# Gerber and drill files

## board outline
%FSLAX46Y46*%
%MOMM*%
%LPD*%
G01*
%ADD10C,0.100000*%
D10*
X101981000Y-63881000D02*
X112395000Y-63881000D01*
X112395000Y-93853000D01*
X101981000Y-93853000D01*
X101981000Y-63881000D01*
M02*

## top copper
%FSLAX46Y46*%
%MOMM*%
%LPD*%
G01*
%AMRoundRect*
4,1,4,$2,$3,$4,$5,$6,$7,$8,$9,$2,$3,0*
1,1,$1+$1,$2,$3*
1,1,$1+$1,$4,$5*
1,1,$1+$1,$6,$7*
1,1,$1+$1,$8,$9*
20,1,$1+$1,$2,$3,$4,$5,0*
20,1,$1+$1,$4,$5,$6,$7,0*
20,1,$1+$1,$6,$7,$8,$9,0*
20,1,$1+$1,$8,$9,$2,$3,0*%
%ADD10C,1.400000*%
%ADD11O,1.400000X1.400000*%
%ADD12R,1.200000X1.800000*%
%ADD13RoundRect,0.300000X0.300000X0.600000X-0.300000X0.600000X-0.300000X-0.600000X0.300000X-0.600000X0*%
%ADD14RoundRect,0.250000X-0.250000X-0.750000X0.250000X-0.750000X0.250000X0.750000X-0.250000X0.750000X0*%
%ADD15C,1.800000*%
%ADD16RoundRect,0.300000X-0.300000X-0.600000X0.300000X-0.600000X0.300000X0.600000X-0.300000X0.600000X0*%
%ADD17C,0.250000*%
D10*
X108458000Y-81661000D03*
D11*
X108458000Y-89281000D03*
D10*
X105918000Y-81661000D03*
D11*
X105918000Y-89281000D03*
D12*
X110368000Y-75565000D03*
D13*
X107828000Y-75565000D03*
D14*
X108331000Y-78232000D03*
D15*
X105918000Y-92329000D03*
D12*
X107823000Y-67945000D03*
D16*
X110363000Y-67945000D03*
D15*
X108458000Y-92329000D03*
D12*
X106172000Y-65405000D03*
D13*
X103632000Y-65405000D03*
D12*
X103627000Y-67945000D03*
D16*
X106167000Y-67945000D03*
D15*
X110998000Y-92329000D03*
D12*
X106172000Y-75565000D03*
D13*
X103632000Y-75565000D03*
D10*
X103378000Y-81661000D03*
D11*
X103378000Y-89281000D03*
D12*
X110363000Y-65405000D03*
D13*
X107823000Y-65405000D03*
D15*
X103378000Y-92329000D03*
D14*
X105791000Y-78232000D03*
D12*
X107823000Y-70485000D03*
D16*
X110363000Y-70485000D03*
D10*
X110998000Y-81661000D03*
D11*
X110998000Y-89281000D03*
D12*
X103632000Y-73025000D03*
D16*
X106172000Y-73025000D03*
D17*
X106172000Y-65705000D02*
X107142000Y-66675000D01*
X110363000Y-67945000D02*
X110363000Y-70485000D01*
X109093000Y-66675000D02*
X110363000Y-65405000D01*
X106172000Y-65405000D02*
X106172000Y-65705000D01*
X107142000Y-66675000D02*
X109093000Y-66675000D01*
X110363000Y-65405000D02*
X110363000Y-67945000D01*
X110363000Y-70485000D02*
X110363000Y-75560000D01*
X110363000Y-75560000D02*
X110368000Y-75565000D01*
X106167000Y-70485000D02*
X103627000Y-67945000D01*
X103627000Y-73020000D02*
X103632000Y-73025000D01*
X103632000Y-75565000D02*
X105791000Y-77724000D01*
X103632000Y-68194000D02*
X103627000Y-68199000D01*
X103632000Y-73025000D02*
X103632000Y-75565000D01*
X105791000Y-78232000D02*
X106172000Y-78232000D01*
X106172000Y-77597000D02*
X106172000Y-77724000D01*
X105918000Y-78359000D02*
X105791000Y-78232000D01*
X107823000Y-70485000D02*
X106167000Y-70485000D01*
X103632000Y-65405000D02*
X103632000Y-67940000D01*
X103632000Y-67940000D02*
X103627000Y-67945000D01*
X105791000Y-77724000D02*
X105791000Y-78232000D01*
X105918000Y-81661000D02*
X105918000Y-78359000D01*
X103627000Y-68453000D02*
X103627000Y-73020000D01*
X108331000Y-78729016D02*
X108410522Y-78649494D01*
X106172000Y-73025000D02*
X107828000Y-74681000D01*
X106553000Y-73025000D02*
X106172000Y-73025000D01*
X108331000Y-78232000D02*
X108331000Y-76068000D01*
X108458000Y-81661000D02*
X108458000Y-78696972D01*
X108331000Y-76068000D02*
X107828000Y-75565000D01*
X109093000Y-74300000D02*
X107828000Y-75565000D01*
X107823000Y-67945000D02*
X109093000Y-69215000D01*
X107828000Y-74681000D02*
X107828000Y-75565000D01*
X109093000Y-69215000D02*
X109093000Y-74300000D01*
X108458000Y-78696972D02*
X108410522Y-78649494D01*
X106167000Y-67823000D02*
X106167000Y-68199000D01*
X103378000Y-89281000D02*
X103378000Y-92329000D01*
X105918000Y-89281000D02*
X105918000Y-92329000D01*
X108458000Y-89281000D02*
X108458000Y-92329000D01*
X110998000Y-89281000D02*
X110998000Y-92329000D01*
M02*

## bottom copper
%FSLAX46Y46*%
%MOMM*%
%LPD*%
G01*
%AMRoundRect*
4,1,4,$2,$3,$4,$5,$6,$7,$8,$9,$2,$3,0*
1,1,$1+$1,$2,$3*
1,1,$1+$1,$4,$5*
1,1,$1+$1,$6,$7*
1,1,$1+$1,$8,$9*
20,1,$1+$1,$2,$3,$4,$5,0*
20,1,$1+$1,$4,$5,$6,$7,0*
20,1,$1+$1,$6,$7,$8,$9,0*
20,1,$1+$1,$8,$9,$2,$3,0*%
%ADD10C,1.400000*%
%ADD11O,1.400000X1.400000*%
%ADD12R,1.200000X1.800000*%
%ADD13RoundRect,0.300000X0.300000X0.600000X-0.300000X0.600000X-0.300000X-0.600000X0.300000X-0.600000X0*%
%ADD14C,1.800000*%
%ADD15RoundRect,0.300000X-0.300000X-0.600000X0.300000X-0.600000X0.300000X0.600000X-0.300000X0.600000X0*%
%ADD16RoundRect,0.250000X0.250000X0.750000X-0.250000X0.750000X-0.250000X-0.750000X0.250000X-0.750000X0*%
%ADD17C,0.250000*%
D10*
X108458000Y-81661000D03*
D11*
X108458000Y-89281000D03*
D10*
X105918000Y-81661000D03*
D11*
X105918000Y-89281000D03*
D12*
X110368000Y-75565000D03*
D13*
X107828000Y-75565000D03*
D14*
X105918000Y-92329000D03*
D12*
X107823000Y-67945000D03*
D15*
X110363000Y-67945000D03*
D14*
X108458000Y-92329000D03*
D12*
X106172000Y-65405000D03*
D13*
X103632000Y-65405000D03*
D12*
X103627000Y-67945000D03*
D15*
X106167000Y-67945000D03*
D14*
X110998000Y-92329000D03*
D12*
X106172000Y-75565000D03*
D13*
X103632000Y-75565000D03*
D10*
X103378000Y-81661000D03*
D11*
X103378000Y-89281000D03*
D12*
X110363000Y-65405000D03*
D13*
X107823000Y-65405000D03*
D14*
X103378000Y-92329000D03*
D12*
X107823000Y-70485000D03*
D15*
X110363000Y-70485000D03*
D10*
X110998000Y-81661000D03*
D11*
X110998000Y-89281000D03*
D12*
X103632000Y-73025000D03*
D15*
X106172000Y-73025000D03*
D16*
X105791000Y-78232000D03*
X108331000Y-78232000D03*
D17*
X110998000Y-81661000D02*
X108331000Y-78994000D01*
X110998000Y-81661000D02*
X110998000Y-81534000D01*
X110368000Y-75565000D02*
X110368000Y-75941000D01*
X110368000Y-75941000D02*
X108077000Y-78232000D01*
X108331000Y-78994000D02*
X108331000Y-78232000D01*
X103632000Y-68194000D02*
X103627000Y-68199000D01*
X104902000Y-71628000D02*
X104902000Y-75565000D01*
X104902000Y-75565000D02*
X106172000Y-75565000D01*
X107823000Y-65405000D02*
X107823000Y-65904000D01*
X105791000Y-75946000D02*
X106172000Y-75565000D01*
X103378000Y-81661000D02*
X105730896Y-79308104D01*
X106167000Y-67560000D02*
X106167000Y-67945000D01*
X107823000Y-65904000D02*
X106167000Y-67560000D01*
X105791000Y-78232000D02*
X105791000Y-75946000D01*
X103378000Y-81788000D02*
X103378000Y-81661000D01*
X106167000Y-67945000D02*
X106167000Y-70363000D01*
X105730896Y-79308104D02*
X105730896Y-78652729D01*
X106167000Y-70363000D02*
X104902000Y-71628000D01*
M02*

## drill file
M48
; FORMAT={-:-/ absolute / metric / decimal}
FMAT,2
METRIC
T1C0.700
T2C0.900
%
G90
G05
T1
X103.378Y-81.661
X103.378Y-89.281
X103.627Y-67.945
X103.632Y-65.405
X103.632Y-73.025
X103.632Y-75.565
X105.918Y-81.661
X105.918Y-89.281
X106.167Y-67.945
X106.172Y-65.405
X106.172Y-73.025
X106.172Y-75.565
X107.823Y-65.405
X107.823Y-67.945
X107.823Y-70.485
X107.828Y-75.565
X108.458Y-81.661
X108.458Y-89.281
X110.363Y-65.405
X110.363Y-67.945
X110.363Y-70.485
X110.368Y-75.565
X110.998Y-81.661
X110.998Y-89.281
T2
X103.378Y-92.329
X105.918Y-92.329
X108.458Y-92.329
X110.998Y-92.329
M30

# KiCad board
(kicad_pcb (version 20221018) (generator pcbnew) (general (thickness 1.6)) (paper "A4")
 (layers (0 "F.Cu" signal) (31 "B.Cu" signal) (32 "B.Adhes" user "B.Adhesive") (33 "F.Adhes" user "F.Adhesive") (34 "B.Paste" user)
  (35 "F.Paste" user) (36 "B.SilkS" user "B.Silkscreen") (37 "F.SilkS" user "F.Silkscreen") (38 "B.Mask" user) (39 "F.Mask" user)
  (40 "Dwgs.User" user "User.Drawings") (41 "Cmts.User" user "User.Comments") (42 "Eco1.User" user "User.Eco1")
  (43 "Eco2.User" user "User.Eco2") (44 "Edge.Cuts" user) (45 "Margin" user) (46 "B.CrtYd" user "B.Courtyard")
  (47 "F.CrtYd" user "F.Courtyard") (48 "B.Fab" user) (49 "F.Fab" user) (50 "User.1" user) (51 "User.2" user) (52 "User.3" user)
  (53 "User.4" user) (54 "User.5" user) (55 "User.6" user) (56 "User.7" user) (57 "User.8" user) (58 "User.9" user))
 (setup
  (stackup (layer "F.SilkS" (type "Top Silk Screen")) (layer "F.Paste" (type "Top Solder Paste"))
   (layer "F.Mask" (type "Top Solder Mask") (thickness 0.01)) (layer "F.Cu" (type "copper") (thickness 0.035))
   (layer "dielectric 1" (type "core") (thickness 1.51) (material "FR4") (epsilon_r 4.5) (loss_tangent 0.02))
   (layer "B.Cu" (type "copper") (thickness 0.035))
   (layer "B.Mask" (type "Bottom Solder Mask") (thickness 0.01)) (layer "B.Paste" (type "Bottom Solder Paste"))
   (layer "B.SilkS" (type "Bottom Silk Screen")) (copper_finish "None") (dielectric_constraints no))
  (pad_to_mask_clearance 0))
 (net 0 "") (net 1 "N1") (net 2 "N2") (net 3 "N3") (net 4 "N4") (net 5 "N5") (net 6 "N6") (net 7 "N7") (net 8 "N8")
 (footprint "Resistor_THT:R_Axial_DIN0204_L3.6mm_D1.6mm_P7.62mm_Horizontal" (layer "F.Cu") (at 108.458 81.661 -90)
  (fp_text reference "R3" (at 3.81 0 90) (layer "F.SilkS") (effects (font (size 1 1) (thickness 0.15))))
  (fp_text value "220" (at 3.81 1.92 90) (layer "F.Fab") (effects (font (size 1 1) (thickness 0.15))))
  (pad "1" thru_hole circle (at 0 0 270) (size 1.4 1.4) (drill 0.7) (layers "*.Cu" "*.Mask") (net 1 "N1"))
  (pad "2" thru_hole oval (at 7.62 0 270) (size 1.4 1.4) (drill 0.7) (layers "*.Cu" "*.Mask") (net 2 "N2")))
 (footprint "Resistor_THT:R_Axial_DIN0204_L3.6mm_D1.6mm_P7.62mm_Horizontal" (layer "F.Cu") (at 105.918 81.661 -90)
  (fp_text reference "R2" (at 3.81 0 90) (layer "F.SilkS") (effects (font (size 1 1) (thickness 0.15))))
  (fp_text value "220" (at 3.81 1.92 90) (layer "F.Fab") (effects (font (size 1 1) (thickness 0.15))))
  (pad "1" thru_hole circle (at 0 0 270) (size 1.4 1.4) (drill 0.7) (layers "*.Cu" "*.Mask") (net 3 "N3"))
  (pad "2" thru_hole oval (at 7.62 0 270) (size 1.4 1.4) (drill 0.7) (layers "*.Cu" "*.Mask") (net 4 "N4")))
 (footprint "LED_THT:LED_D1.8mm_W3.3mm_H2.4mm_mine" (layer "F.Cu") (at 110.368 75.565 180)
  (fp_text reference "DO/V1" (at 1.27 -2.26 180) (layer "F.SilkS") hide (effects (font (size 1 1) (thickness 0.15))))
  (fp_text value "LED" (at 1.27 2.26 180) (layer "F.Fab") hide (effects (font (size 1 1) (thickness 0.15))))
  (pad "1" thru_hole rect (at 0 0 180) (size 1.2 1.8) (drill 0.7) (layers "*.Cu" "*.Mask") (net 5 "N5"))
  (pad "2" thru_hole roundrect (at 2.54 0 180) (size 1.2 1.8) (drill 0.7) (layers "*.Cu" "*.Mask") (roundrect_rratio 0.25) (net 1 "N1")))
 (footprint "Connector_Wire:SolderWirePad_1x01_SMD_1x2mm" (layer "F.Cu") (at 108.331 78.232)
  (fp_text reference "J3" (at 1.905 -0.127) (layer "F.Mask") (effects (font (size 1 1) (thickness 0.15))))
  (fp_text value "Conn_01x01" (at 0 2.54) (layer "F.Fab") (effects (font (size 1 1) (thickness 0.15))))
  (pad "1" smd roundrect (at 0 0) (size 1 2) (layers "F.Cu" "F.Paste" "F.Mask") (roundrect_rratio 0.25) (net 1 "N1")))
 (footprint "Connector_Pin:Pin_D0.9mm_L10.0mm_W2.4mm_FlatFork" (layer "F.Cu") (at 105.918 92.329)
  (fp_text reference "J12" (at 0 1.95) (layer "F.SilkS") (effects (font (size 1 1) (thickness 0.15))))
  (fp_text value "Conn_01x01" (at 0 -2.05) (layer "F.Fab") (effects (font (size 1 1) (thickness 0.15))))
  (pad "1" thru_hole circle (at 0 0) (size 1.8 1.8) (drill 0.9) (layers "*.Cu" "*.Mask") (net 4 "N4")))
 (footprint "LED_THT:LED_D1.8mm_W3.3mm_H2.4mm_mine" (layer "F.Cu") (at 107.823 67.945)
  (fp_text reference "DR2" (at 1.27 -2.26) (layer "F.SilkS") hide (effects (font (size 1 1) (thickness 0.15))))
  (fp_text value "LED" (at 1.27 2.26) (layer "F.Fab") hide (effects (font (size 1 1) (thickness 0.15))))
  (pad "1" thru_hole rect (at 0 0) (size 1.2 1.8) (drill 0.7) (layers "*.Cu" "*.Mask") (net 1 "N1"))
  (pad "2" thru_hole roundrect (at 2.54 0) (size 1.2 1.8) (drill 0.7) (layers "*.Cu" "*.Mask") (roundrect_rratio 0.25) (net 5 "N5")))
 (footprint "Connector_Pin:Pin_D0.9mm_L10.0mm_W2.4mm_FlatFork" (layer "F.Cu") (at 108.458 92.329)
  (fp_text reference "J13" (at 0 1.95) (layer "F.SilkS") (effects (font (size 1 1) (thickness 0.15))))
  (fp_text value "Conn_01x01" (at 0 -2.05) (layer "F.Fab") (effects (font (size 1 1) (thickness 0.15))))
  (pad "1" thru_hole circle (at 0 0) (size 1.8 1.8) (drill 0.9) (layers "*.Cu" "*.Mask") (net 2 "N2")))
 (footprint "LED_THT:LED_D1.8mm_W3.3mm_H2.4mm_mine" (layer "F.Cu") (at 106.172 65.405 180)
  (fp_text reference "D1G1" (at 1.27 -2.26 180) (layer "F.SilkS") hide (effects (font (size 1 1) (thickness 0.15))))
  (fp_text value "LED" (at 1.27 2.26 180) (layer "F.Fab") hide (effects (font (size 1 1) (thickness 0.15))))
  (pad "1" thru_hole rect (at 0 0 180) (size 1.2 1.8) (drill 0.7) (layers "*.Cu" "*.Mask") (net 5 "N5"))
  (pad "2" thru_hole roundrect (at 2.54 0 180) (size 1.2 1.8) (drill 0.7) (layers "*.Cu" "*.Mask") (roundrect_rratio 0.25) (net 3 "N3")))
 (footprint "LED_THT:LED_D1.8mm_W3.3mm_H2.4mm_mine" (layer "F.Cu") (at 103.627 67.945)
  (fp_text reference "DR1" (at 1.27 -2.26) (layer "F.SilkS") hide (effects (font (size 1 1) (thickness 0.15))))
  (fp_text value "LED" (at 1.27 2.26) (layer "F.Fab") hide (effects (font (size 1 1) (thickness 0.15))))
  (pad "1" thru_hole rect (at 0 0) (size 1.2 1.8) (drill 0.7) (layers "*.Cu" "*.Mask") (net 3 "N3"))
  (pad "2" thru_hole roundrect (at 2.54 0) (size 1.2 1.8) (drill 0.7) (layers "*.Cu" "*.Mask") (roundrect_rratio 0.25) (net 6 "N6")))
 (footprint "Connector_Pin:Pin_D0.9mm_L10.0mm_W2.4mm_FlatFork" (layer "F.Cu") (at 110.998 92.329)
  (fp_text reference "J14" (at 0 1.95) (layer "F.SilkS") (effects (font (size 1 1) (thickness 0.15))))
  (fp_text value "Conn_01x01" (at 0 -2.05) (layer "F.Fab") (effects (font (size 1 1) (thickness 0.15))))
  (pad "1" thru_hole circle (at 0 0) (size 1.8 1.8) (drill 0.9) (layers "*.Cu" "*.Mask") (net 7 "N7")))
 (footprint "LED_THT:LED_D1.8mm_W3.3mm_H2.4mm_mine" (layer "F.Cu") (at 106.172 75.565 180)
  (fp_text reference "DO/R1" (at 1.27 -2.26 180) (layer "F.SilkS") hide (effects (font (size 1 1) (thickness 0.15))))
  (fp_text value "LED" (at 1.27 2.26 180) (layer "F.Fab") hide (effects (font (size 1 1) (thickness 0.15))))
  (pad "1" thru_hole rect (at 0 0 180) (size 1.2 1.8) (drill 0.7) (layers "*.Cu" "*.Mask") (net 6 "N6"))
  (pad "2" thru_hole roundrect (at 2.54 0 180) (size 1.2 1.8) (drill 0.7) (layers "*.Cu" "*.Mask") (roundrect_rratio 0.25) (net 3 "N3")))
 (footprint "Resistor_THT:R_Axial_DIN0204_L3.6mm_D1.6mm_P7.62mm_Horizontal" (layer "F.Cu") (at 103.378 81.661 -90)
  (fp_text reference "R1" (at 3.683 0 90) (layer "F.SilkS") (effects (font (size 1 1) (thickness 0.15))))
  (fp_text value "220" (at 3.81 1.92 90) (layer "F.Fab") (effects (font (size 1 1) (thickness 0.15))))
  (pad "1" thru_hole circle (at 0 0 270) (size 1.4 1.4) (drill 0.7) (layers "*.Cu" "*.Mask") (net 6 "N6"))
  (pad "2" thru_hole oval (at 7.62 0 270) (size 1.4 1.4) (drill 0.7) (layers "*.Cu" "*.Mask") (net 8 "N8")))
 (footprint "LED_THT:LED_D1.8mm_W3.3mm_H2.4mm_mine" (layer "F.Cu") (at 110.363 65.405 180)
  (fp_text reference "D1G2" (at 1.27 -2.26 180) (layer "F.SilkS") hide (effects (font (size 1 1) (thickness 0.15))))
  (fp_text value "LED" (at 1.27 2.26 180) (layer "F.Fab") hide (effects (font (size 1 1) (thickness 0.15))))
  (pad "1" thru_hole rect (at 0 0 180) (size 1.2 1.8) (drill 0.7) (layers "*.Cu" "*.Mask") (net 5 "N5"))
  (pad "2" thru_hole roundrect (at 2.54 0 180) (size 1.2 1.8) (drill 0.7) (layers "*.Cu" "*.Mask") (roundrect_rratio 0.25) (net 6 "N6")))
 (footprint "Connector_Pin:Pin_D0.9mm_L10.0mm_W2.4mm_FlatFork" (layer "F.Cu") (at 103.378 92.329)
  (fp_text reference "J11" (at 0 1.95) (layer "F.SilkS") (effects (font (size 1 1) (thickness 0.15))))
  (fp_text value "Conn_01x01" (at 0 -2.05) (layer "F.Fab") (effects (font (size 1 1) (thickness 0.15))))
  (pad "1" thru_hole circle (at 0 0) (size 1.8 1.8) (drill 0.9) (layers "*.Cu" "*.Mask") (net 8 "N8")))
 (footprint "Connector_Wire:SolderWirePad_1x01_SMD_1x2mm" (layer "F.Cu") (at 105.791 78.232)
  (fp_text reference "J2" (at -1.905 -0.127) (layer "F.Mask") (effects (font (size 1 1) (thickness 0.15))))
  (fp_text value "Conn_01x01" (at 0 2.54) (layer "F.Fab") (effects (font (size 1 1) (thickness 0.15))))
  (pad "1" smd roundrect (at 0 0) (size 1 2) (layers "F.Cu" "F.Paste" "F.Mask") (roundrect_rratio 0.25) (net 3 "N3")))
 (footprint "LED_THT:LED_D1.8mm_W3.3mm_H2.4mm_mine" (layer "F.Cu") (at 107.823 70.485)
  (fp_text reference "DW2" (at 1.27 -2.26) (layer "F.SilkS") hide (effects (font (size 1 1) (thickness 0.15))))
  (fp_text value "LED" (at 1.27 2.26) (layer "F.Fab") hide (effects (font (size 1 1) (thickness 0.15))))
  (pad "1" thru_hole rect (at 0 0) (size 1.2 1.8) (drill 0.7) (layers "*.Cu" "*.Mask") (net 3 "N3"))
  (pad "2" thru_hole roundrect (at 2.54 0) (size 1.2 1.8) (drill 0.7) (layers "*.Cu" "*.Mask") (roundrect_rratio 0.25) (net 5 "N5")))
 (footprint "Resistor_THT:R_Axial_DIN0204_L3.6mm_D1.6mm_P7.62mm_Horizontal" (layer "F.Cu") (at 110.998 81.661 -90)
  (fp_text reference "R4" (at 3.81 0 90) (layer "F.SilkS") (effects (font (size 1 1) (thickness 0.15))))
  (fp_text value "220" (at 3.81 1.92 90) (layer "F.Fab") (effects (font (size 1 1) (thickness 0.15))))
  (pad "1" thru_hole circle (at 0 0 270) (size 1.4 1.4) (drill 0.7) (layers "*.Cu" "*.Mask") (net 5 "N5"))
  (pad "2" thru_hole oval (at 7.62 0 270) (size 1.4 1.4) (drill 0.7) (layers "*.Cu" "*.Mask") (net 7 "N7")))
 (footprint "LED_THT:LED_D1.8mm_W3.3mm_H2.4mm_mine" (layer "F.Cu") (at 103.632 73.025)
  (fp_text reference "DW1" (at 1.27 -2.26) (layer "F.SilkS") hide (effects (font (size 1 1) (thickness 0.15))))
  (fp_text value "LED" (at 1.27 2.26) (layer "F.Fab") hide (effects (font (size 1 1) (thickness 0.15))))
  (pad "1" thru_hole rect (at 0 0) (size 1.2 1.8) (drill 0.7) (layers "*.Cu" "*.Mask") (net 3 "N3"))
  (pad "2" thru_hole roundrect (at 2.54 0) (size 1.2 1.8) (drill 0.7) (layers "*.Cu" "*.Mask") (roundrect_rratio 0.25) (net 1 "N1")))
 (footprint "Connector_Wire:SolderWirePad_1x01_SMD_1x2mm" (layer "B.Cu") (at 105.791 78.232 180)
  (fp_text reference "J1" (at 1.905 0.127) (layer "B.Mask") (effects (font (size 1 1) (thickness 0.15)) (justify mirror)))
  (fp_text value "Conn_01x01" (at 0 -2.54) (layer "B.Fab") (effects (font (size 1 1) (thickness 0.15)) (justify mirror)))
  (pad "1" smd roundrect (at 0 0 180) (size 1 2) (layers "B.Cu" "B.Paste" "B.Mask") (roundrect_rratio 0.25) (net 6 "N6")))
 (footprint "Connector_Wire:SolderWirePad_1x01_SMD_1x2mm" (layer "B.Cu") (at 108.331 78.232 180)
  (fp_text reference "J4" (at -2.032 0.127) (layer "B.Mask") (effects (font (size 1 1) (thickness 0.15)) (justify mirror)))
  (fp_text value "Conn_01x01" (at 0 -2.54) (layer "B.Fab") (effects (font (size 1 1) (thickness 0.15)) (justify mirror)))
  (pad "1" smd roundrect (at 0 0 180) (size 1 2) (layers "B.Cu" "B.Paste" "B.Mask") (roundrect_rratio 0.25) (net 5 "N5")))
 (gr_rect (start 101.981 63.881) (end 112.395 93.853) (stroke (width 0.1) (type default)) (fill none) (layer "Edge.Cuts"))
 (segment (start 106.172 65.705) (end 107.142 66.675) (width 0.25) (layer "F.Cu") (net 5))
 (segment (start 110.363 67.945) (end 110.363 70.485) (width 0.25) (layer "F.Cu") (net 5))
 (segment (start 109.093 66.675) (end 110.363 65.405) (width 0.25) (layer "F.Cu") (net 5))
 (segment (start 106.172 65.405) (end 106.172 65.705) (width 0.25) (layer "F.Cu") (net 5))
 (segment (start 107.142 66.675) (end 109.093 66.675) (width 0.25) (layer "F.Cu") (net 5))
 (segment (start 110.363 65.405) (end 110.363 67.945) (width 0.25) (layer "F.Cu") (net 5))
 (segment (start 110.363 70.485) (end 110.363 75.56) (width 0.25) (layer "F.Cu") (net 5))
 (segment (start 110.363 75.56) (end 110.368 75.565) (width 0.25) (layer "F.Cu") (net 5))
 (segment (start 110.998 81.661) (end 108.331 78.994) (width 0.25) (layer "B.Cu") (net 5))
 (segment (start 110.998 81.661) (end 110.998 81.534) (width 0.25) (layer "B.Cu") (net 5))
 (segment (start 110.368 75.565) (end 110.368 75.941) (width 0.25) (layer "B.Cu") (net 5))
 (segment (start 110.368 75.941) (end 108.077 78.232) (width 0.25) (layer "B.Cu") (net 5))
 (segment (start 108.331 78.994) (end 108.331 78.232) (width 0.25) (layer "B.Cu") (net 5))
 (segment (start 106.167 70.485) (end 103.627 67.945) (width 0.25) (layer "F.Cu") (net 3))
 (segment (start 103.627 73.02) (end 103.632 73.025) (width 0.25) (layer "F.Cu") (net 3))
 (segment (start 103.632 75.565) (end 105.791 77.724) (width 0.25) (layer "F.Cu") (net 3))
 (segment (start 103.632 68.194) (end 103.627 68.199) (width 0.25) (layer "F.Cu") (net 3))
 (segment (start 103.632 73.025) (end 103.632 75.565) (width 0.25) (layer "F.Cu") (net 3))
 (segment (start 105.791 78.232) (end 106.172 78.232) (width 0.25) (layer "F.Cu") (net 3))
 (segment (start 106.172 77.597) (end 106.172 77.724) (width 0.25) (layer "F.Cu") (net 3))
 (segment (start 105.918 78.359) (end 105.791 78.232) (width 0.25) (layer "F.Cu") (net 3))
 (segment (start 107.823 70.485) (end 106.167 70.485) (width 0.25) (layer "F.Cu") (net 3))
 (segment (start 103.632 65.405) (end 103.632 67.94) (width 0.25) (layer "F.Cu") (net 3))
 (segment (start 103.632 67.94) (end 103.627 67.945) (width 0.25) (layer "F.Cu") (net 3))
 (segment (start 105.791 77.724) (end 105.791 78.232) (width 0.25) (layer "F.Cu") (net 3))
 (segment (start 105.918 81.661) (end 105.918 78.359) (width 0.25) (layer "F.Cu") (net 3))
 (segment (start 103.627 68.453) (end 103.627 73.02) (width 0.25) (layer "F.Cu") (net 3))
 (segment (start 103.632 68.194) (end 103.627 68.199) (width 0.25) (layer "B.Cu") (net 3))
 (segment (start 108.331 78.729016) (end 108.410522 78.649494) (width 0.25) (layer "F.Cu") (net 1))
 (segment (start 106.172 73.025) (end 107.828 74.681) (width 0.25) (layer "F.Cu") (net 1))
 (segment (start 106.553 73.025) (end 106.172 73.025) (width 0.25) (layer "F.Cu") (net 1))
 (segment (start 108.331 78.232) (end 108.331 76.068) (width 0.25) (layer "F.Cu") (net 1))
 (segment (start 108.458 81.661) (end 108.458 78.696972) (width 0.25) (layer "F.Cu") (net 1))
 (segment (start 108.331 76.068) (end 107.828 75.565) (width 0.25) (layer "F.Cu") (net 1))
 (segment (start 109.093 74.3) (end 107.828 75.565) (width 0.25) (layer "F.Cu") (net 1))
 (segment (start 107.823 67.945) (end 109.093 69.215) (width 0.25) (layer "F.Cu") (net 1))
 (segment (start 107.828 74.681) (end 107.828 75.565) (width 0.25) (layer "F.Cu") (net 1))
 (segment (start 109.093 69.215) (end 109.093 74.3) (width 0.25) (layer "F.Cu") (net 1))
 (segment (start 108.458 78.696972) (end 108.410522 78.649494) (width 0.25) (layer "F.Cu") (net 1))
 (segment (start 106.167 67.823) (end 106.167 68.199) (width 0.25) (layer "F.Cu") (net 6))
 (segment (start 104.902 71.628) (end 104.902 75.565) (width 0.25) (layer "B.Cu") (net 6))
 (segment (start 104.902 75.565) (end 106.172 75.565) (width 0.25) (layer "B.Cu") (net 6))
 (segment (start 107.823 65.405) (end 107.823 65.904) (width 0.25) (layer "B.Cu") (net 6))
 (segment (start 105.791 75.946) (end 106.172 75.565) (width 0.25) (layer "B.Cu") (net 6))
 (segment (start 103.378 81.661) (end 105.730896 79.308104) (width 0.25) (layer "B.Cu") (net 6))
 (segment (start 106.167 67.56) (end 106.167 67.945) (width 0.25) (layer "B.Cu") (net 6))
 (segment (start 107.823 65.904) (end 106.167 67.56) (width 0.25) (layer "B.Cu") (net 6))
 (segment (start 105.791 78.232) (end 105.791 75.946) (width 0.25) (layer "B.Cu") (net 6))
 (segment (start 103.378 81.788) (end 103.378 81.661) (width 0.25) (layer "B.Cu") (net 6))
 (segment (start 106.167 67.945) (end 106.167 70.363) (width 0.25) (layer "B.Cu") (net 6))
 (segment (start 105.730896 79.308104) (end 105.730896 78.652729) (width 0.25) (layer "B.Cu") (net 6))
 (segment (start 106.167 70.363) (end 104.902 71.628) (width 0.25) (layer "B.Cu") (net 6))
 (segment (start 103.378 89.281) (end 103.378 92.329) (width 0.25) (layer "F.Cu") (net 8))
 (segment (start 105.918 89.281) (end 105.918 92.329) (width 0.25) (layer "F.Cu") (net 4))
 (segment (start 108.458 89.281) (end 108.458 92.329) (width 0.25) (layer "F.Cu") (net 2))
 (segment (start 110.998 89.281) (end 110.998 92.329) (width 0.25) (layer "F.Cu") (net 7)))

